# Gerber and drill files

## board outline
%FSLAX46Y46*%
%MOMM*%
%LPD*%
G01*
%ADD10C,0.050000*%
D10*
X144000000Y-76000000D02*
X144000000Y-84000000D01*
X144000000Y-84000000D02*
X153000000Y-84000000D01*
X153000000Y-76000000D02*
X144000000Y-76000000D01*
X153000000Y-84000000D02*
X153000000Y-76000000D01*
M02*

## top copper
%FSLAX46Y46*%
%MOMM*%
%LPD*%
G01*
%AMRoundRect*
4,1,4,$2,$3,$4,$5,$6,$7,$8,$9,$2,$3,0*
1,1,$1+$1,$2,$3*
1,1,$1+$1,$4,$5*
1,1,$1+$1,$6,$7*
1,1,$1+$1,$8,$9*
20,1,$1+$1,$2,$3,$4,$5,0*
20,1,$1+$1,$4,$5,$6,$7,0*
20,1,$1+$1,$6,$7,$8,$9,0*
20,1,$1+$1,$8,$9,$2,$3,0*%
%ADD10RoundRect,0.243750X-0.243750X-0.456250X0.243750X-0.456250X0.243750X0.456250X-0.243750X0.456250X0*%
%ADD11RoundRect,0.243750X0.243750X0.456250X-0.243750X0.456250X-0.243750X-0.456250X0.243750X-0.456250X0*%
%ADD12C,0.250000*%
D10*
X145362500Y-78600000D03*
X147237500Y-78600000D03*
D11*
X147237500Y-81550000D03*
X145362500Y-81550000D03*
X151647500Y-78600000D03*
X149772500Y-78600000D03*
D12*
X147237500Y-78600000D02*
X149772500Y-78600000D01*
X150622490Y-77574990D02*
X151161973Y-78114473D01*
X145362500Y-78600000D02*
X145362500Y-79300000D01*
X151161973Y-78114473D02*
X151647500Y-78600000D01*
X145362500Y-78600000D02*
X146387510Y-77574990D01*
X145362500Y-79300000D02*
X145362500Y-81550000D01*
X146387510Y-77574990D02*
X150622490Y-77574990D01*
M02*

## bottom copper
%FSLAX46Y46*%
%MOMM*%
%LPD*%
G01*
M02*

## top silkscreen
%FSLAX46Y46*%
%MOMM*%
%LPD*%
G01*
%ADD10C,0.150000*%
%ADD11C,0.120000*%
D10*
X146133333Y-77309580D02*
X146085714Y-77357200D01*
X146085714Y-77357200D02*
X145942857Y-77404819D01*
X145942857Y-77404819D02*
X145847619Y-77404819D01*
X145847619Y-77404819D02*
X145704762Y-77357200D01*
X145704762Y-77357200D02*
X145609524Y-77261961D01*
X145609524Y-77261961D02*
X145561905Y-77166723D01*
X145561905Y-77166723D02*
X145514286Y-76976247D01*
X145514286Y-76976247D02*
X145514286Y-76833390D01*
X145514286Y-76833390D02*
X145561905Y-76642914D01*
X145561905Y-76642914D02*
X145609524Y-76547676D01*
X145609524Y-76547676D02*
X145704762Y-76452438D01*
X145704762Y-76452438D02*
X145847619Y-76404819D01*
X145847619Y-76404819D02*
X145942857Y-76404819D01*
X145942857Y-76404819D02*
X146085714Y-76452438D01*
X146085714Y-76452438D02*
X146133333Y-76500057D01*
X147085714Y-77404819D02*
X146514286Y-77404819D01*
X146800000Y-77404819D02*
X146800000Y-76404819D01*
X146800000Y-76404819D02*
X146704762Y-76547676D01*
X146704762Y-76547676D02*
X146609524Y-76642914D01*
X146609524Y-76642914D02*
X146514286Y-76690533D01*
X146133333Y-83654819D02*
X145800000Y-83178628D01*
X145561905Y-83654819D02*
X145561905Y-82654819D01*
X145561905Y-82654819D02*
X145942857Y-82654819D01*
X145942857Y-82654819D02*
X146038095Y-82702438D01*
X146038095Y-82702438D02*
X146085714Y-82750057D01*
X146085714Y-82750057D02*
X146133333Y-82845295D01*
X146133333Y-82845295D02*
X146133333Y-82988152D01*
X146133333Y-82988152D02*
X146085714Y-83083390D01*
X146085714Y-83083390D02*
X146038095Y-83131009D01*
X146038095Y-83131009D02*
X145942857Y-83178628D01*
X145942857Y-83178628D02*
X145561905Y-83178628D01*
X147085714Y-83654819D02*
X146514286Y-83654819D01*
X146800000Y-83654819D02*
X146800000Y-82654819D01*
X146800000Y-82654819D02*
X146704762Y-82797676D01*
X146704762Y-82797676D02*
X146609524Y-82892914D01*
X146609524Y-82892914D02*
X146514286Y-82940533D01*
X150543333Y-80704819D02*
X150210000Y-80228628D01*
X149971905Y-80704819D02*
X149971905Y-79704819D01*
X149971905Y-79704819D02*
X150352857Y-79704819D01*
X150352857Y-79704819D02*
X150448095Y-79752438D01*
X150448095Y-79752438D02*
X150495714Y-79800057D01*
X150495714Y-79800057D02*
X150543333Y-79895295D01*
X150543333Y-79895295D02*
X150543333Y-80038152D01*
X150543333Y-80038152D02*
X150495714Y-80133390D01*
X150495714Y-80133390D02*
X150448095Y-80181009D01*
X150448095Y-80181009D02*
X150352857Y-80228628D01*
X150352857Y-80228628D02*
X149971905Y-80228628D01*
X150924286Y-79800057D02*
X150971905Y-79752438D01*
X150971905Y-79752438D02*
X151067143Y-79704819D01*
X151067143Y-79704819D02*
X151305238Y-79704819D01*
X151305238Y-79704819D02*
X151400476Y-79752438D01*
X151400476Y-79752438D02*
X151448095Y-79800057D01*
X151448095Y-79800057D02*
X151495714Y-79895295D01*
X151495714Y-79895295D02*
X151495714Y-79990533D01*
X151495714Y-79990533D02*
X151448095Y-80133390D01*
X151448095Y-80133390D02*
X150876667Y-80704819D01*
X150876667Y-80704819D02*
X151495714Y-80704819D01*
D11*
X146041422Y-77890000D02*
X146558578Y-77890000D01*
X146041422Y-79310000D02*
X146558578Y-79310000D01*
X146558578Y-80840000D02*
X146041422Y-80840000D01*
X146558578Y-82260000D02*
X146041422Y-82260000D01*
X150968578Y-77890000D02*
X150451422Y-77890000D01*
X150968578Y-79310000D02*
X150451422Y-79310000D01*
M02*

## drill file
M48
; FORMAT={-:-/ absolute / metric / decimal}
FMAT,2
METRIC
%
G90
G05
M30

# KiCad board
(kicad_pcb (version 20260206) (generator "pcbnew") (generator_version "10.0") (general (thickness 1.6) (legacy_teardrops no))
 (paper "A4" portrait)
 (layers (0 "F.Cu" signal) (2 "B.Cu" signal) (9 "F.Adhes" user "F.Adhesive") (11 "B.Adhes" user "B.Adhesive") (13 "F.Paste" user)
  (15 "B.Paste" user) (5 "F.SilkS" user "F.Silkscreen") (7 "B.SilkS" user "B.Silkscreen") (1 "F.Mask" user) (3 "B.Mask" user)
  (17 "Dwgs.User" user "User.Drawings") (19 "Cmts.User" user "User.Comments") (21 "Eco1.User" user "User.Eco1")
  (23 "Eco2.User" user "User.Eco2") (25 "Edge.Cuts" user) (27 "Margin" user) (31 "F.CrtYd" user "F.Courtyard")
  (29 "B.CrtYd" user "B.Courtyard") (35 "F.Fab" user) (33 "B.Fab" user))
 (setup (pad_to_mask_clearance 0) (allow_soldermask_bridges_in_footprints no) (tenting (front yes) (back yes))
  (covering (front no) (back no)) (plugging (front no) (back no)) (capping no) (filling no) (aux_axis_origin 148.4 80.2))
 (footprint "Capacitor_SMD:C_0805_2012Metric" (layer "F.Cu") (at 146.3 78.6)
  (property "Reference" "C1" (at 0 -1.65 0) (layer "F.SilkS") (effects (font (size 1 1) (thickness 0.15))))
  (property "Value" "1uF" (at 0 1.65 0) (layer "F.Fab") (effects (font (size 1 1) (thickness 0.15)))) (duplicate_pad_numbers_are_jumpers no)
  (fp_line (start -0.258578 -0.71) (end 0.258578 -0.71) (stroke (width 0.12) (type solid)) (layer "F.SilkS"))
  (fp_line (start -0.258578 0.71) (end 0.258578 0.71) (stroke (width 0.12) (type solid)) (layer "F.SilkS"))
  (pad "1" smd roundrect (at -0.9375 0) (size 0.975 1.4) (layers "F.Cu" "F.Mask" "F.Paste") (roundrect_rratio 0.25) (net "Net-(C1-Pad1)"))
  (pad "2" smd roundrect (at 0.9375 0) (size 0.975 1.4) (layers "F.Cu" "F.Mask" "F.Paste") (roundrect_rratio 0.25) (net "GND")))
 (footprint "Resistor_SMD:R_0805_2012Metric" (layer "F.Cu") (at 146.3 81.55 180)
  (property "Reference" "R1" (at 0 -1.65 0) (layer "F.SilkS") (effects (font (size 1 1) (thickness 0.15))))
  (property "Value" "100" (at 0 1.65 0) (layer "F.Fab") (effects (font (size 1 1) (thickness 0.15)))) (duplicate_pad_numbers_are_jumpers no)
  (fp_line (start -0.258578 0.71) (end 0.258578 0.71) (stroke (width 0.12) (type solid)) (layer "F.SilkS"))
  (fp_line (start -0.258578 -0.71) (end 0.258578 -0.71) (stroke (width 0.12) (type solid)) (layer "F.SilkS"))
  (pad "1" smd roundrect (at -0.9375 0 180) (size 0.975 1.4) (layers "F.Cu" "F.Mask" "F.Paste") (roundrect_rratio 0.25) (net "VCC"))
  (pad "2" smd roundrect (at 0.9375 0 180) (size 0.975 1.4) (layers "F.Cu" "F.Mask" "F.Paste") (roundrect_rratio 0.25) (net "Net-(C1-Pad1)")))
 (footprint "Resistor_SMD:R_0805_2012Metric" (layer "F.Cu") (at 150.71 78.6 180)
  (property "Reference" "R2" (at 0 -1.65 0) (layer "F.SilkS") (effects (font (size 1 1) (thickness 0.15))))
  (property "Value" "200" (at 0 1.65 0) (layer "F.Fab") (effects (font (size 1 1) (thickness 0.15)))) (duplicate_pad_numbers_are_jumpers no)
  (fp_line (start -0.258578 0.71) (end 0.258578 0.71) (stroke (width 0.12) (type solid)) (layer "F.SilkS"))
  (fp_line (start -0.258578 -0.71) (end 0.258578 -0.71) (stroke (width 0.12) (type solid)) (layer "F.SilkS"))
  (pad "1" smd roundrect (at -0.9375 0 180) (size 0.975 1.4) (layers "F.Cu" "F.Mask" "F.Paste") (roundrect_rratio 0.25)
   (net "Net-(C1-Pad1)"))
  (pad "2" smd roundrect (at 0.9375 0 180) (size 0.975 1.4) (layers "F.Cu" "F.Mask" "F.Paste") (roundrect_rratio 0.25) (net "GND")))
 (gr_line (start 144 76) (end 144 84) (stroke (width 0.05) (type solid)) (layer "Edge.Cuts"))
 (gr_line (start 144 84) (end 153 84) (stroke (width 0.05) (type solid)) (layer "Edge.Cuts"))
 (gr_line (start 153 76) (end 144 76) (stroke (width 0.05) (type solid)) (layer "Edge.Cuts"))
 (gr_line (start 153 84) (end 153 76) (stroke (width 0.05) (type solid)) (layer "Edge.Cuts"))
 (segment (start 147.2375 78.6) (end 149.7725 78.6) (width 0.25) (layer "F.Cu") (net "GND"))
 (segment (start 150.62249 77.57499) (end 151.161973 78.114473) (width 0.25) (layer "F.Cu") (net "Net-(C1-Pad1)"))
 (segment (start 145.3625 78.6) (end 145.3625 79.3) (width 0.25) (layer "F.Cu") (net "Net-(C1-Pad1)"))
 (segment (start 151.161973 78.114473) (end 151.6475 78.6) (width 0.25) (layer "F.Cu") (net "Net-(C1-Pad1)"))
 (segment (start 145.3625 78.6) (end 146.38751 77.57499) (width 0.25) (layer "F.Cu") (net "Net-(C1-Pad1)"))
 (segment (start 145.3625 79.3) (end 145.3625 81.55) (width 0.25) (layer "F.Cu") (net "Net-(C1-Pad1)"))
 (segment (start 146.38751 77.57499) (end 150.62249 77.57499) (width 0.25) (layer "F.Cu") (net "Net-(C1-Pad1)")))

